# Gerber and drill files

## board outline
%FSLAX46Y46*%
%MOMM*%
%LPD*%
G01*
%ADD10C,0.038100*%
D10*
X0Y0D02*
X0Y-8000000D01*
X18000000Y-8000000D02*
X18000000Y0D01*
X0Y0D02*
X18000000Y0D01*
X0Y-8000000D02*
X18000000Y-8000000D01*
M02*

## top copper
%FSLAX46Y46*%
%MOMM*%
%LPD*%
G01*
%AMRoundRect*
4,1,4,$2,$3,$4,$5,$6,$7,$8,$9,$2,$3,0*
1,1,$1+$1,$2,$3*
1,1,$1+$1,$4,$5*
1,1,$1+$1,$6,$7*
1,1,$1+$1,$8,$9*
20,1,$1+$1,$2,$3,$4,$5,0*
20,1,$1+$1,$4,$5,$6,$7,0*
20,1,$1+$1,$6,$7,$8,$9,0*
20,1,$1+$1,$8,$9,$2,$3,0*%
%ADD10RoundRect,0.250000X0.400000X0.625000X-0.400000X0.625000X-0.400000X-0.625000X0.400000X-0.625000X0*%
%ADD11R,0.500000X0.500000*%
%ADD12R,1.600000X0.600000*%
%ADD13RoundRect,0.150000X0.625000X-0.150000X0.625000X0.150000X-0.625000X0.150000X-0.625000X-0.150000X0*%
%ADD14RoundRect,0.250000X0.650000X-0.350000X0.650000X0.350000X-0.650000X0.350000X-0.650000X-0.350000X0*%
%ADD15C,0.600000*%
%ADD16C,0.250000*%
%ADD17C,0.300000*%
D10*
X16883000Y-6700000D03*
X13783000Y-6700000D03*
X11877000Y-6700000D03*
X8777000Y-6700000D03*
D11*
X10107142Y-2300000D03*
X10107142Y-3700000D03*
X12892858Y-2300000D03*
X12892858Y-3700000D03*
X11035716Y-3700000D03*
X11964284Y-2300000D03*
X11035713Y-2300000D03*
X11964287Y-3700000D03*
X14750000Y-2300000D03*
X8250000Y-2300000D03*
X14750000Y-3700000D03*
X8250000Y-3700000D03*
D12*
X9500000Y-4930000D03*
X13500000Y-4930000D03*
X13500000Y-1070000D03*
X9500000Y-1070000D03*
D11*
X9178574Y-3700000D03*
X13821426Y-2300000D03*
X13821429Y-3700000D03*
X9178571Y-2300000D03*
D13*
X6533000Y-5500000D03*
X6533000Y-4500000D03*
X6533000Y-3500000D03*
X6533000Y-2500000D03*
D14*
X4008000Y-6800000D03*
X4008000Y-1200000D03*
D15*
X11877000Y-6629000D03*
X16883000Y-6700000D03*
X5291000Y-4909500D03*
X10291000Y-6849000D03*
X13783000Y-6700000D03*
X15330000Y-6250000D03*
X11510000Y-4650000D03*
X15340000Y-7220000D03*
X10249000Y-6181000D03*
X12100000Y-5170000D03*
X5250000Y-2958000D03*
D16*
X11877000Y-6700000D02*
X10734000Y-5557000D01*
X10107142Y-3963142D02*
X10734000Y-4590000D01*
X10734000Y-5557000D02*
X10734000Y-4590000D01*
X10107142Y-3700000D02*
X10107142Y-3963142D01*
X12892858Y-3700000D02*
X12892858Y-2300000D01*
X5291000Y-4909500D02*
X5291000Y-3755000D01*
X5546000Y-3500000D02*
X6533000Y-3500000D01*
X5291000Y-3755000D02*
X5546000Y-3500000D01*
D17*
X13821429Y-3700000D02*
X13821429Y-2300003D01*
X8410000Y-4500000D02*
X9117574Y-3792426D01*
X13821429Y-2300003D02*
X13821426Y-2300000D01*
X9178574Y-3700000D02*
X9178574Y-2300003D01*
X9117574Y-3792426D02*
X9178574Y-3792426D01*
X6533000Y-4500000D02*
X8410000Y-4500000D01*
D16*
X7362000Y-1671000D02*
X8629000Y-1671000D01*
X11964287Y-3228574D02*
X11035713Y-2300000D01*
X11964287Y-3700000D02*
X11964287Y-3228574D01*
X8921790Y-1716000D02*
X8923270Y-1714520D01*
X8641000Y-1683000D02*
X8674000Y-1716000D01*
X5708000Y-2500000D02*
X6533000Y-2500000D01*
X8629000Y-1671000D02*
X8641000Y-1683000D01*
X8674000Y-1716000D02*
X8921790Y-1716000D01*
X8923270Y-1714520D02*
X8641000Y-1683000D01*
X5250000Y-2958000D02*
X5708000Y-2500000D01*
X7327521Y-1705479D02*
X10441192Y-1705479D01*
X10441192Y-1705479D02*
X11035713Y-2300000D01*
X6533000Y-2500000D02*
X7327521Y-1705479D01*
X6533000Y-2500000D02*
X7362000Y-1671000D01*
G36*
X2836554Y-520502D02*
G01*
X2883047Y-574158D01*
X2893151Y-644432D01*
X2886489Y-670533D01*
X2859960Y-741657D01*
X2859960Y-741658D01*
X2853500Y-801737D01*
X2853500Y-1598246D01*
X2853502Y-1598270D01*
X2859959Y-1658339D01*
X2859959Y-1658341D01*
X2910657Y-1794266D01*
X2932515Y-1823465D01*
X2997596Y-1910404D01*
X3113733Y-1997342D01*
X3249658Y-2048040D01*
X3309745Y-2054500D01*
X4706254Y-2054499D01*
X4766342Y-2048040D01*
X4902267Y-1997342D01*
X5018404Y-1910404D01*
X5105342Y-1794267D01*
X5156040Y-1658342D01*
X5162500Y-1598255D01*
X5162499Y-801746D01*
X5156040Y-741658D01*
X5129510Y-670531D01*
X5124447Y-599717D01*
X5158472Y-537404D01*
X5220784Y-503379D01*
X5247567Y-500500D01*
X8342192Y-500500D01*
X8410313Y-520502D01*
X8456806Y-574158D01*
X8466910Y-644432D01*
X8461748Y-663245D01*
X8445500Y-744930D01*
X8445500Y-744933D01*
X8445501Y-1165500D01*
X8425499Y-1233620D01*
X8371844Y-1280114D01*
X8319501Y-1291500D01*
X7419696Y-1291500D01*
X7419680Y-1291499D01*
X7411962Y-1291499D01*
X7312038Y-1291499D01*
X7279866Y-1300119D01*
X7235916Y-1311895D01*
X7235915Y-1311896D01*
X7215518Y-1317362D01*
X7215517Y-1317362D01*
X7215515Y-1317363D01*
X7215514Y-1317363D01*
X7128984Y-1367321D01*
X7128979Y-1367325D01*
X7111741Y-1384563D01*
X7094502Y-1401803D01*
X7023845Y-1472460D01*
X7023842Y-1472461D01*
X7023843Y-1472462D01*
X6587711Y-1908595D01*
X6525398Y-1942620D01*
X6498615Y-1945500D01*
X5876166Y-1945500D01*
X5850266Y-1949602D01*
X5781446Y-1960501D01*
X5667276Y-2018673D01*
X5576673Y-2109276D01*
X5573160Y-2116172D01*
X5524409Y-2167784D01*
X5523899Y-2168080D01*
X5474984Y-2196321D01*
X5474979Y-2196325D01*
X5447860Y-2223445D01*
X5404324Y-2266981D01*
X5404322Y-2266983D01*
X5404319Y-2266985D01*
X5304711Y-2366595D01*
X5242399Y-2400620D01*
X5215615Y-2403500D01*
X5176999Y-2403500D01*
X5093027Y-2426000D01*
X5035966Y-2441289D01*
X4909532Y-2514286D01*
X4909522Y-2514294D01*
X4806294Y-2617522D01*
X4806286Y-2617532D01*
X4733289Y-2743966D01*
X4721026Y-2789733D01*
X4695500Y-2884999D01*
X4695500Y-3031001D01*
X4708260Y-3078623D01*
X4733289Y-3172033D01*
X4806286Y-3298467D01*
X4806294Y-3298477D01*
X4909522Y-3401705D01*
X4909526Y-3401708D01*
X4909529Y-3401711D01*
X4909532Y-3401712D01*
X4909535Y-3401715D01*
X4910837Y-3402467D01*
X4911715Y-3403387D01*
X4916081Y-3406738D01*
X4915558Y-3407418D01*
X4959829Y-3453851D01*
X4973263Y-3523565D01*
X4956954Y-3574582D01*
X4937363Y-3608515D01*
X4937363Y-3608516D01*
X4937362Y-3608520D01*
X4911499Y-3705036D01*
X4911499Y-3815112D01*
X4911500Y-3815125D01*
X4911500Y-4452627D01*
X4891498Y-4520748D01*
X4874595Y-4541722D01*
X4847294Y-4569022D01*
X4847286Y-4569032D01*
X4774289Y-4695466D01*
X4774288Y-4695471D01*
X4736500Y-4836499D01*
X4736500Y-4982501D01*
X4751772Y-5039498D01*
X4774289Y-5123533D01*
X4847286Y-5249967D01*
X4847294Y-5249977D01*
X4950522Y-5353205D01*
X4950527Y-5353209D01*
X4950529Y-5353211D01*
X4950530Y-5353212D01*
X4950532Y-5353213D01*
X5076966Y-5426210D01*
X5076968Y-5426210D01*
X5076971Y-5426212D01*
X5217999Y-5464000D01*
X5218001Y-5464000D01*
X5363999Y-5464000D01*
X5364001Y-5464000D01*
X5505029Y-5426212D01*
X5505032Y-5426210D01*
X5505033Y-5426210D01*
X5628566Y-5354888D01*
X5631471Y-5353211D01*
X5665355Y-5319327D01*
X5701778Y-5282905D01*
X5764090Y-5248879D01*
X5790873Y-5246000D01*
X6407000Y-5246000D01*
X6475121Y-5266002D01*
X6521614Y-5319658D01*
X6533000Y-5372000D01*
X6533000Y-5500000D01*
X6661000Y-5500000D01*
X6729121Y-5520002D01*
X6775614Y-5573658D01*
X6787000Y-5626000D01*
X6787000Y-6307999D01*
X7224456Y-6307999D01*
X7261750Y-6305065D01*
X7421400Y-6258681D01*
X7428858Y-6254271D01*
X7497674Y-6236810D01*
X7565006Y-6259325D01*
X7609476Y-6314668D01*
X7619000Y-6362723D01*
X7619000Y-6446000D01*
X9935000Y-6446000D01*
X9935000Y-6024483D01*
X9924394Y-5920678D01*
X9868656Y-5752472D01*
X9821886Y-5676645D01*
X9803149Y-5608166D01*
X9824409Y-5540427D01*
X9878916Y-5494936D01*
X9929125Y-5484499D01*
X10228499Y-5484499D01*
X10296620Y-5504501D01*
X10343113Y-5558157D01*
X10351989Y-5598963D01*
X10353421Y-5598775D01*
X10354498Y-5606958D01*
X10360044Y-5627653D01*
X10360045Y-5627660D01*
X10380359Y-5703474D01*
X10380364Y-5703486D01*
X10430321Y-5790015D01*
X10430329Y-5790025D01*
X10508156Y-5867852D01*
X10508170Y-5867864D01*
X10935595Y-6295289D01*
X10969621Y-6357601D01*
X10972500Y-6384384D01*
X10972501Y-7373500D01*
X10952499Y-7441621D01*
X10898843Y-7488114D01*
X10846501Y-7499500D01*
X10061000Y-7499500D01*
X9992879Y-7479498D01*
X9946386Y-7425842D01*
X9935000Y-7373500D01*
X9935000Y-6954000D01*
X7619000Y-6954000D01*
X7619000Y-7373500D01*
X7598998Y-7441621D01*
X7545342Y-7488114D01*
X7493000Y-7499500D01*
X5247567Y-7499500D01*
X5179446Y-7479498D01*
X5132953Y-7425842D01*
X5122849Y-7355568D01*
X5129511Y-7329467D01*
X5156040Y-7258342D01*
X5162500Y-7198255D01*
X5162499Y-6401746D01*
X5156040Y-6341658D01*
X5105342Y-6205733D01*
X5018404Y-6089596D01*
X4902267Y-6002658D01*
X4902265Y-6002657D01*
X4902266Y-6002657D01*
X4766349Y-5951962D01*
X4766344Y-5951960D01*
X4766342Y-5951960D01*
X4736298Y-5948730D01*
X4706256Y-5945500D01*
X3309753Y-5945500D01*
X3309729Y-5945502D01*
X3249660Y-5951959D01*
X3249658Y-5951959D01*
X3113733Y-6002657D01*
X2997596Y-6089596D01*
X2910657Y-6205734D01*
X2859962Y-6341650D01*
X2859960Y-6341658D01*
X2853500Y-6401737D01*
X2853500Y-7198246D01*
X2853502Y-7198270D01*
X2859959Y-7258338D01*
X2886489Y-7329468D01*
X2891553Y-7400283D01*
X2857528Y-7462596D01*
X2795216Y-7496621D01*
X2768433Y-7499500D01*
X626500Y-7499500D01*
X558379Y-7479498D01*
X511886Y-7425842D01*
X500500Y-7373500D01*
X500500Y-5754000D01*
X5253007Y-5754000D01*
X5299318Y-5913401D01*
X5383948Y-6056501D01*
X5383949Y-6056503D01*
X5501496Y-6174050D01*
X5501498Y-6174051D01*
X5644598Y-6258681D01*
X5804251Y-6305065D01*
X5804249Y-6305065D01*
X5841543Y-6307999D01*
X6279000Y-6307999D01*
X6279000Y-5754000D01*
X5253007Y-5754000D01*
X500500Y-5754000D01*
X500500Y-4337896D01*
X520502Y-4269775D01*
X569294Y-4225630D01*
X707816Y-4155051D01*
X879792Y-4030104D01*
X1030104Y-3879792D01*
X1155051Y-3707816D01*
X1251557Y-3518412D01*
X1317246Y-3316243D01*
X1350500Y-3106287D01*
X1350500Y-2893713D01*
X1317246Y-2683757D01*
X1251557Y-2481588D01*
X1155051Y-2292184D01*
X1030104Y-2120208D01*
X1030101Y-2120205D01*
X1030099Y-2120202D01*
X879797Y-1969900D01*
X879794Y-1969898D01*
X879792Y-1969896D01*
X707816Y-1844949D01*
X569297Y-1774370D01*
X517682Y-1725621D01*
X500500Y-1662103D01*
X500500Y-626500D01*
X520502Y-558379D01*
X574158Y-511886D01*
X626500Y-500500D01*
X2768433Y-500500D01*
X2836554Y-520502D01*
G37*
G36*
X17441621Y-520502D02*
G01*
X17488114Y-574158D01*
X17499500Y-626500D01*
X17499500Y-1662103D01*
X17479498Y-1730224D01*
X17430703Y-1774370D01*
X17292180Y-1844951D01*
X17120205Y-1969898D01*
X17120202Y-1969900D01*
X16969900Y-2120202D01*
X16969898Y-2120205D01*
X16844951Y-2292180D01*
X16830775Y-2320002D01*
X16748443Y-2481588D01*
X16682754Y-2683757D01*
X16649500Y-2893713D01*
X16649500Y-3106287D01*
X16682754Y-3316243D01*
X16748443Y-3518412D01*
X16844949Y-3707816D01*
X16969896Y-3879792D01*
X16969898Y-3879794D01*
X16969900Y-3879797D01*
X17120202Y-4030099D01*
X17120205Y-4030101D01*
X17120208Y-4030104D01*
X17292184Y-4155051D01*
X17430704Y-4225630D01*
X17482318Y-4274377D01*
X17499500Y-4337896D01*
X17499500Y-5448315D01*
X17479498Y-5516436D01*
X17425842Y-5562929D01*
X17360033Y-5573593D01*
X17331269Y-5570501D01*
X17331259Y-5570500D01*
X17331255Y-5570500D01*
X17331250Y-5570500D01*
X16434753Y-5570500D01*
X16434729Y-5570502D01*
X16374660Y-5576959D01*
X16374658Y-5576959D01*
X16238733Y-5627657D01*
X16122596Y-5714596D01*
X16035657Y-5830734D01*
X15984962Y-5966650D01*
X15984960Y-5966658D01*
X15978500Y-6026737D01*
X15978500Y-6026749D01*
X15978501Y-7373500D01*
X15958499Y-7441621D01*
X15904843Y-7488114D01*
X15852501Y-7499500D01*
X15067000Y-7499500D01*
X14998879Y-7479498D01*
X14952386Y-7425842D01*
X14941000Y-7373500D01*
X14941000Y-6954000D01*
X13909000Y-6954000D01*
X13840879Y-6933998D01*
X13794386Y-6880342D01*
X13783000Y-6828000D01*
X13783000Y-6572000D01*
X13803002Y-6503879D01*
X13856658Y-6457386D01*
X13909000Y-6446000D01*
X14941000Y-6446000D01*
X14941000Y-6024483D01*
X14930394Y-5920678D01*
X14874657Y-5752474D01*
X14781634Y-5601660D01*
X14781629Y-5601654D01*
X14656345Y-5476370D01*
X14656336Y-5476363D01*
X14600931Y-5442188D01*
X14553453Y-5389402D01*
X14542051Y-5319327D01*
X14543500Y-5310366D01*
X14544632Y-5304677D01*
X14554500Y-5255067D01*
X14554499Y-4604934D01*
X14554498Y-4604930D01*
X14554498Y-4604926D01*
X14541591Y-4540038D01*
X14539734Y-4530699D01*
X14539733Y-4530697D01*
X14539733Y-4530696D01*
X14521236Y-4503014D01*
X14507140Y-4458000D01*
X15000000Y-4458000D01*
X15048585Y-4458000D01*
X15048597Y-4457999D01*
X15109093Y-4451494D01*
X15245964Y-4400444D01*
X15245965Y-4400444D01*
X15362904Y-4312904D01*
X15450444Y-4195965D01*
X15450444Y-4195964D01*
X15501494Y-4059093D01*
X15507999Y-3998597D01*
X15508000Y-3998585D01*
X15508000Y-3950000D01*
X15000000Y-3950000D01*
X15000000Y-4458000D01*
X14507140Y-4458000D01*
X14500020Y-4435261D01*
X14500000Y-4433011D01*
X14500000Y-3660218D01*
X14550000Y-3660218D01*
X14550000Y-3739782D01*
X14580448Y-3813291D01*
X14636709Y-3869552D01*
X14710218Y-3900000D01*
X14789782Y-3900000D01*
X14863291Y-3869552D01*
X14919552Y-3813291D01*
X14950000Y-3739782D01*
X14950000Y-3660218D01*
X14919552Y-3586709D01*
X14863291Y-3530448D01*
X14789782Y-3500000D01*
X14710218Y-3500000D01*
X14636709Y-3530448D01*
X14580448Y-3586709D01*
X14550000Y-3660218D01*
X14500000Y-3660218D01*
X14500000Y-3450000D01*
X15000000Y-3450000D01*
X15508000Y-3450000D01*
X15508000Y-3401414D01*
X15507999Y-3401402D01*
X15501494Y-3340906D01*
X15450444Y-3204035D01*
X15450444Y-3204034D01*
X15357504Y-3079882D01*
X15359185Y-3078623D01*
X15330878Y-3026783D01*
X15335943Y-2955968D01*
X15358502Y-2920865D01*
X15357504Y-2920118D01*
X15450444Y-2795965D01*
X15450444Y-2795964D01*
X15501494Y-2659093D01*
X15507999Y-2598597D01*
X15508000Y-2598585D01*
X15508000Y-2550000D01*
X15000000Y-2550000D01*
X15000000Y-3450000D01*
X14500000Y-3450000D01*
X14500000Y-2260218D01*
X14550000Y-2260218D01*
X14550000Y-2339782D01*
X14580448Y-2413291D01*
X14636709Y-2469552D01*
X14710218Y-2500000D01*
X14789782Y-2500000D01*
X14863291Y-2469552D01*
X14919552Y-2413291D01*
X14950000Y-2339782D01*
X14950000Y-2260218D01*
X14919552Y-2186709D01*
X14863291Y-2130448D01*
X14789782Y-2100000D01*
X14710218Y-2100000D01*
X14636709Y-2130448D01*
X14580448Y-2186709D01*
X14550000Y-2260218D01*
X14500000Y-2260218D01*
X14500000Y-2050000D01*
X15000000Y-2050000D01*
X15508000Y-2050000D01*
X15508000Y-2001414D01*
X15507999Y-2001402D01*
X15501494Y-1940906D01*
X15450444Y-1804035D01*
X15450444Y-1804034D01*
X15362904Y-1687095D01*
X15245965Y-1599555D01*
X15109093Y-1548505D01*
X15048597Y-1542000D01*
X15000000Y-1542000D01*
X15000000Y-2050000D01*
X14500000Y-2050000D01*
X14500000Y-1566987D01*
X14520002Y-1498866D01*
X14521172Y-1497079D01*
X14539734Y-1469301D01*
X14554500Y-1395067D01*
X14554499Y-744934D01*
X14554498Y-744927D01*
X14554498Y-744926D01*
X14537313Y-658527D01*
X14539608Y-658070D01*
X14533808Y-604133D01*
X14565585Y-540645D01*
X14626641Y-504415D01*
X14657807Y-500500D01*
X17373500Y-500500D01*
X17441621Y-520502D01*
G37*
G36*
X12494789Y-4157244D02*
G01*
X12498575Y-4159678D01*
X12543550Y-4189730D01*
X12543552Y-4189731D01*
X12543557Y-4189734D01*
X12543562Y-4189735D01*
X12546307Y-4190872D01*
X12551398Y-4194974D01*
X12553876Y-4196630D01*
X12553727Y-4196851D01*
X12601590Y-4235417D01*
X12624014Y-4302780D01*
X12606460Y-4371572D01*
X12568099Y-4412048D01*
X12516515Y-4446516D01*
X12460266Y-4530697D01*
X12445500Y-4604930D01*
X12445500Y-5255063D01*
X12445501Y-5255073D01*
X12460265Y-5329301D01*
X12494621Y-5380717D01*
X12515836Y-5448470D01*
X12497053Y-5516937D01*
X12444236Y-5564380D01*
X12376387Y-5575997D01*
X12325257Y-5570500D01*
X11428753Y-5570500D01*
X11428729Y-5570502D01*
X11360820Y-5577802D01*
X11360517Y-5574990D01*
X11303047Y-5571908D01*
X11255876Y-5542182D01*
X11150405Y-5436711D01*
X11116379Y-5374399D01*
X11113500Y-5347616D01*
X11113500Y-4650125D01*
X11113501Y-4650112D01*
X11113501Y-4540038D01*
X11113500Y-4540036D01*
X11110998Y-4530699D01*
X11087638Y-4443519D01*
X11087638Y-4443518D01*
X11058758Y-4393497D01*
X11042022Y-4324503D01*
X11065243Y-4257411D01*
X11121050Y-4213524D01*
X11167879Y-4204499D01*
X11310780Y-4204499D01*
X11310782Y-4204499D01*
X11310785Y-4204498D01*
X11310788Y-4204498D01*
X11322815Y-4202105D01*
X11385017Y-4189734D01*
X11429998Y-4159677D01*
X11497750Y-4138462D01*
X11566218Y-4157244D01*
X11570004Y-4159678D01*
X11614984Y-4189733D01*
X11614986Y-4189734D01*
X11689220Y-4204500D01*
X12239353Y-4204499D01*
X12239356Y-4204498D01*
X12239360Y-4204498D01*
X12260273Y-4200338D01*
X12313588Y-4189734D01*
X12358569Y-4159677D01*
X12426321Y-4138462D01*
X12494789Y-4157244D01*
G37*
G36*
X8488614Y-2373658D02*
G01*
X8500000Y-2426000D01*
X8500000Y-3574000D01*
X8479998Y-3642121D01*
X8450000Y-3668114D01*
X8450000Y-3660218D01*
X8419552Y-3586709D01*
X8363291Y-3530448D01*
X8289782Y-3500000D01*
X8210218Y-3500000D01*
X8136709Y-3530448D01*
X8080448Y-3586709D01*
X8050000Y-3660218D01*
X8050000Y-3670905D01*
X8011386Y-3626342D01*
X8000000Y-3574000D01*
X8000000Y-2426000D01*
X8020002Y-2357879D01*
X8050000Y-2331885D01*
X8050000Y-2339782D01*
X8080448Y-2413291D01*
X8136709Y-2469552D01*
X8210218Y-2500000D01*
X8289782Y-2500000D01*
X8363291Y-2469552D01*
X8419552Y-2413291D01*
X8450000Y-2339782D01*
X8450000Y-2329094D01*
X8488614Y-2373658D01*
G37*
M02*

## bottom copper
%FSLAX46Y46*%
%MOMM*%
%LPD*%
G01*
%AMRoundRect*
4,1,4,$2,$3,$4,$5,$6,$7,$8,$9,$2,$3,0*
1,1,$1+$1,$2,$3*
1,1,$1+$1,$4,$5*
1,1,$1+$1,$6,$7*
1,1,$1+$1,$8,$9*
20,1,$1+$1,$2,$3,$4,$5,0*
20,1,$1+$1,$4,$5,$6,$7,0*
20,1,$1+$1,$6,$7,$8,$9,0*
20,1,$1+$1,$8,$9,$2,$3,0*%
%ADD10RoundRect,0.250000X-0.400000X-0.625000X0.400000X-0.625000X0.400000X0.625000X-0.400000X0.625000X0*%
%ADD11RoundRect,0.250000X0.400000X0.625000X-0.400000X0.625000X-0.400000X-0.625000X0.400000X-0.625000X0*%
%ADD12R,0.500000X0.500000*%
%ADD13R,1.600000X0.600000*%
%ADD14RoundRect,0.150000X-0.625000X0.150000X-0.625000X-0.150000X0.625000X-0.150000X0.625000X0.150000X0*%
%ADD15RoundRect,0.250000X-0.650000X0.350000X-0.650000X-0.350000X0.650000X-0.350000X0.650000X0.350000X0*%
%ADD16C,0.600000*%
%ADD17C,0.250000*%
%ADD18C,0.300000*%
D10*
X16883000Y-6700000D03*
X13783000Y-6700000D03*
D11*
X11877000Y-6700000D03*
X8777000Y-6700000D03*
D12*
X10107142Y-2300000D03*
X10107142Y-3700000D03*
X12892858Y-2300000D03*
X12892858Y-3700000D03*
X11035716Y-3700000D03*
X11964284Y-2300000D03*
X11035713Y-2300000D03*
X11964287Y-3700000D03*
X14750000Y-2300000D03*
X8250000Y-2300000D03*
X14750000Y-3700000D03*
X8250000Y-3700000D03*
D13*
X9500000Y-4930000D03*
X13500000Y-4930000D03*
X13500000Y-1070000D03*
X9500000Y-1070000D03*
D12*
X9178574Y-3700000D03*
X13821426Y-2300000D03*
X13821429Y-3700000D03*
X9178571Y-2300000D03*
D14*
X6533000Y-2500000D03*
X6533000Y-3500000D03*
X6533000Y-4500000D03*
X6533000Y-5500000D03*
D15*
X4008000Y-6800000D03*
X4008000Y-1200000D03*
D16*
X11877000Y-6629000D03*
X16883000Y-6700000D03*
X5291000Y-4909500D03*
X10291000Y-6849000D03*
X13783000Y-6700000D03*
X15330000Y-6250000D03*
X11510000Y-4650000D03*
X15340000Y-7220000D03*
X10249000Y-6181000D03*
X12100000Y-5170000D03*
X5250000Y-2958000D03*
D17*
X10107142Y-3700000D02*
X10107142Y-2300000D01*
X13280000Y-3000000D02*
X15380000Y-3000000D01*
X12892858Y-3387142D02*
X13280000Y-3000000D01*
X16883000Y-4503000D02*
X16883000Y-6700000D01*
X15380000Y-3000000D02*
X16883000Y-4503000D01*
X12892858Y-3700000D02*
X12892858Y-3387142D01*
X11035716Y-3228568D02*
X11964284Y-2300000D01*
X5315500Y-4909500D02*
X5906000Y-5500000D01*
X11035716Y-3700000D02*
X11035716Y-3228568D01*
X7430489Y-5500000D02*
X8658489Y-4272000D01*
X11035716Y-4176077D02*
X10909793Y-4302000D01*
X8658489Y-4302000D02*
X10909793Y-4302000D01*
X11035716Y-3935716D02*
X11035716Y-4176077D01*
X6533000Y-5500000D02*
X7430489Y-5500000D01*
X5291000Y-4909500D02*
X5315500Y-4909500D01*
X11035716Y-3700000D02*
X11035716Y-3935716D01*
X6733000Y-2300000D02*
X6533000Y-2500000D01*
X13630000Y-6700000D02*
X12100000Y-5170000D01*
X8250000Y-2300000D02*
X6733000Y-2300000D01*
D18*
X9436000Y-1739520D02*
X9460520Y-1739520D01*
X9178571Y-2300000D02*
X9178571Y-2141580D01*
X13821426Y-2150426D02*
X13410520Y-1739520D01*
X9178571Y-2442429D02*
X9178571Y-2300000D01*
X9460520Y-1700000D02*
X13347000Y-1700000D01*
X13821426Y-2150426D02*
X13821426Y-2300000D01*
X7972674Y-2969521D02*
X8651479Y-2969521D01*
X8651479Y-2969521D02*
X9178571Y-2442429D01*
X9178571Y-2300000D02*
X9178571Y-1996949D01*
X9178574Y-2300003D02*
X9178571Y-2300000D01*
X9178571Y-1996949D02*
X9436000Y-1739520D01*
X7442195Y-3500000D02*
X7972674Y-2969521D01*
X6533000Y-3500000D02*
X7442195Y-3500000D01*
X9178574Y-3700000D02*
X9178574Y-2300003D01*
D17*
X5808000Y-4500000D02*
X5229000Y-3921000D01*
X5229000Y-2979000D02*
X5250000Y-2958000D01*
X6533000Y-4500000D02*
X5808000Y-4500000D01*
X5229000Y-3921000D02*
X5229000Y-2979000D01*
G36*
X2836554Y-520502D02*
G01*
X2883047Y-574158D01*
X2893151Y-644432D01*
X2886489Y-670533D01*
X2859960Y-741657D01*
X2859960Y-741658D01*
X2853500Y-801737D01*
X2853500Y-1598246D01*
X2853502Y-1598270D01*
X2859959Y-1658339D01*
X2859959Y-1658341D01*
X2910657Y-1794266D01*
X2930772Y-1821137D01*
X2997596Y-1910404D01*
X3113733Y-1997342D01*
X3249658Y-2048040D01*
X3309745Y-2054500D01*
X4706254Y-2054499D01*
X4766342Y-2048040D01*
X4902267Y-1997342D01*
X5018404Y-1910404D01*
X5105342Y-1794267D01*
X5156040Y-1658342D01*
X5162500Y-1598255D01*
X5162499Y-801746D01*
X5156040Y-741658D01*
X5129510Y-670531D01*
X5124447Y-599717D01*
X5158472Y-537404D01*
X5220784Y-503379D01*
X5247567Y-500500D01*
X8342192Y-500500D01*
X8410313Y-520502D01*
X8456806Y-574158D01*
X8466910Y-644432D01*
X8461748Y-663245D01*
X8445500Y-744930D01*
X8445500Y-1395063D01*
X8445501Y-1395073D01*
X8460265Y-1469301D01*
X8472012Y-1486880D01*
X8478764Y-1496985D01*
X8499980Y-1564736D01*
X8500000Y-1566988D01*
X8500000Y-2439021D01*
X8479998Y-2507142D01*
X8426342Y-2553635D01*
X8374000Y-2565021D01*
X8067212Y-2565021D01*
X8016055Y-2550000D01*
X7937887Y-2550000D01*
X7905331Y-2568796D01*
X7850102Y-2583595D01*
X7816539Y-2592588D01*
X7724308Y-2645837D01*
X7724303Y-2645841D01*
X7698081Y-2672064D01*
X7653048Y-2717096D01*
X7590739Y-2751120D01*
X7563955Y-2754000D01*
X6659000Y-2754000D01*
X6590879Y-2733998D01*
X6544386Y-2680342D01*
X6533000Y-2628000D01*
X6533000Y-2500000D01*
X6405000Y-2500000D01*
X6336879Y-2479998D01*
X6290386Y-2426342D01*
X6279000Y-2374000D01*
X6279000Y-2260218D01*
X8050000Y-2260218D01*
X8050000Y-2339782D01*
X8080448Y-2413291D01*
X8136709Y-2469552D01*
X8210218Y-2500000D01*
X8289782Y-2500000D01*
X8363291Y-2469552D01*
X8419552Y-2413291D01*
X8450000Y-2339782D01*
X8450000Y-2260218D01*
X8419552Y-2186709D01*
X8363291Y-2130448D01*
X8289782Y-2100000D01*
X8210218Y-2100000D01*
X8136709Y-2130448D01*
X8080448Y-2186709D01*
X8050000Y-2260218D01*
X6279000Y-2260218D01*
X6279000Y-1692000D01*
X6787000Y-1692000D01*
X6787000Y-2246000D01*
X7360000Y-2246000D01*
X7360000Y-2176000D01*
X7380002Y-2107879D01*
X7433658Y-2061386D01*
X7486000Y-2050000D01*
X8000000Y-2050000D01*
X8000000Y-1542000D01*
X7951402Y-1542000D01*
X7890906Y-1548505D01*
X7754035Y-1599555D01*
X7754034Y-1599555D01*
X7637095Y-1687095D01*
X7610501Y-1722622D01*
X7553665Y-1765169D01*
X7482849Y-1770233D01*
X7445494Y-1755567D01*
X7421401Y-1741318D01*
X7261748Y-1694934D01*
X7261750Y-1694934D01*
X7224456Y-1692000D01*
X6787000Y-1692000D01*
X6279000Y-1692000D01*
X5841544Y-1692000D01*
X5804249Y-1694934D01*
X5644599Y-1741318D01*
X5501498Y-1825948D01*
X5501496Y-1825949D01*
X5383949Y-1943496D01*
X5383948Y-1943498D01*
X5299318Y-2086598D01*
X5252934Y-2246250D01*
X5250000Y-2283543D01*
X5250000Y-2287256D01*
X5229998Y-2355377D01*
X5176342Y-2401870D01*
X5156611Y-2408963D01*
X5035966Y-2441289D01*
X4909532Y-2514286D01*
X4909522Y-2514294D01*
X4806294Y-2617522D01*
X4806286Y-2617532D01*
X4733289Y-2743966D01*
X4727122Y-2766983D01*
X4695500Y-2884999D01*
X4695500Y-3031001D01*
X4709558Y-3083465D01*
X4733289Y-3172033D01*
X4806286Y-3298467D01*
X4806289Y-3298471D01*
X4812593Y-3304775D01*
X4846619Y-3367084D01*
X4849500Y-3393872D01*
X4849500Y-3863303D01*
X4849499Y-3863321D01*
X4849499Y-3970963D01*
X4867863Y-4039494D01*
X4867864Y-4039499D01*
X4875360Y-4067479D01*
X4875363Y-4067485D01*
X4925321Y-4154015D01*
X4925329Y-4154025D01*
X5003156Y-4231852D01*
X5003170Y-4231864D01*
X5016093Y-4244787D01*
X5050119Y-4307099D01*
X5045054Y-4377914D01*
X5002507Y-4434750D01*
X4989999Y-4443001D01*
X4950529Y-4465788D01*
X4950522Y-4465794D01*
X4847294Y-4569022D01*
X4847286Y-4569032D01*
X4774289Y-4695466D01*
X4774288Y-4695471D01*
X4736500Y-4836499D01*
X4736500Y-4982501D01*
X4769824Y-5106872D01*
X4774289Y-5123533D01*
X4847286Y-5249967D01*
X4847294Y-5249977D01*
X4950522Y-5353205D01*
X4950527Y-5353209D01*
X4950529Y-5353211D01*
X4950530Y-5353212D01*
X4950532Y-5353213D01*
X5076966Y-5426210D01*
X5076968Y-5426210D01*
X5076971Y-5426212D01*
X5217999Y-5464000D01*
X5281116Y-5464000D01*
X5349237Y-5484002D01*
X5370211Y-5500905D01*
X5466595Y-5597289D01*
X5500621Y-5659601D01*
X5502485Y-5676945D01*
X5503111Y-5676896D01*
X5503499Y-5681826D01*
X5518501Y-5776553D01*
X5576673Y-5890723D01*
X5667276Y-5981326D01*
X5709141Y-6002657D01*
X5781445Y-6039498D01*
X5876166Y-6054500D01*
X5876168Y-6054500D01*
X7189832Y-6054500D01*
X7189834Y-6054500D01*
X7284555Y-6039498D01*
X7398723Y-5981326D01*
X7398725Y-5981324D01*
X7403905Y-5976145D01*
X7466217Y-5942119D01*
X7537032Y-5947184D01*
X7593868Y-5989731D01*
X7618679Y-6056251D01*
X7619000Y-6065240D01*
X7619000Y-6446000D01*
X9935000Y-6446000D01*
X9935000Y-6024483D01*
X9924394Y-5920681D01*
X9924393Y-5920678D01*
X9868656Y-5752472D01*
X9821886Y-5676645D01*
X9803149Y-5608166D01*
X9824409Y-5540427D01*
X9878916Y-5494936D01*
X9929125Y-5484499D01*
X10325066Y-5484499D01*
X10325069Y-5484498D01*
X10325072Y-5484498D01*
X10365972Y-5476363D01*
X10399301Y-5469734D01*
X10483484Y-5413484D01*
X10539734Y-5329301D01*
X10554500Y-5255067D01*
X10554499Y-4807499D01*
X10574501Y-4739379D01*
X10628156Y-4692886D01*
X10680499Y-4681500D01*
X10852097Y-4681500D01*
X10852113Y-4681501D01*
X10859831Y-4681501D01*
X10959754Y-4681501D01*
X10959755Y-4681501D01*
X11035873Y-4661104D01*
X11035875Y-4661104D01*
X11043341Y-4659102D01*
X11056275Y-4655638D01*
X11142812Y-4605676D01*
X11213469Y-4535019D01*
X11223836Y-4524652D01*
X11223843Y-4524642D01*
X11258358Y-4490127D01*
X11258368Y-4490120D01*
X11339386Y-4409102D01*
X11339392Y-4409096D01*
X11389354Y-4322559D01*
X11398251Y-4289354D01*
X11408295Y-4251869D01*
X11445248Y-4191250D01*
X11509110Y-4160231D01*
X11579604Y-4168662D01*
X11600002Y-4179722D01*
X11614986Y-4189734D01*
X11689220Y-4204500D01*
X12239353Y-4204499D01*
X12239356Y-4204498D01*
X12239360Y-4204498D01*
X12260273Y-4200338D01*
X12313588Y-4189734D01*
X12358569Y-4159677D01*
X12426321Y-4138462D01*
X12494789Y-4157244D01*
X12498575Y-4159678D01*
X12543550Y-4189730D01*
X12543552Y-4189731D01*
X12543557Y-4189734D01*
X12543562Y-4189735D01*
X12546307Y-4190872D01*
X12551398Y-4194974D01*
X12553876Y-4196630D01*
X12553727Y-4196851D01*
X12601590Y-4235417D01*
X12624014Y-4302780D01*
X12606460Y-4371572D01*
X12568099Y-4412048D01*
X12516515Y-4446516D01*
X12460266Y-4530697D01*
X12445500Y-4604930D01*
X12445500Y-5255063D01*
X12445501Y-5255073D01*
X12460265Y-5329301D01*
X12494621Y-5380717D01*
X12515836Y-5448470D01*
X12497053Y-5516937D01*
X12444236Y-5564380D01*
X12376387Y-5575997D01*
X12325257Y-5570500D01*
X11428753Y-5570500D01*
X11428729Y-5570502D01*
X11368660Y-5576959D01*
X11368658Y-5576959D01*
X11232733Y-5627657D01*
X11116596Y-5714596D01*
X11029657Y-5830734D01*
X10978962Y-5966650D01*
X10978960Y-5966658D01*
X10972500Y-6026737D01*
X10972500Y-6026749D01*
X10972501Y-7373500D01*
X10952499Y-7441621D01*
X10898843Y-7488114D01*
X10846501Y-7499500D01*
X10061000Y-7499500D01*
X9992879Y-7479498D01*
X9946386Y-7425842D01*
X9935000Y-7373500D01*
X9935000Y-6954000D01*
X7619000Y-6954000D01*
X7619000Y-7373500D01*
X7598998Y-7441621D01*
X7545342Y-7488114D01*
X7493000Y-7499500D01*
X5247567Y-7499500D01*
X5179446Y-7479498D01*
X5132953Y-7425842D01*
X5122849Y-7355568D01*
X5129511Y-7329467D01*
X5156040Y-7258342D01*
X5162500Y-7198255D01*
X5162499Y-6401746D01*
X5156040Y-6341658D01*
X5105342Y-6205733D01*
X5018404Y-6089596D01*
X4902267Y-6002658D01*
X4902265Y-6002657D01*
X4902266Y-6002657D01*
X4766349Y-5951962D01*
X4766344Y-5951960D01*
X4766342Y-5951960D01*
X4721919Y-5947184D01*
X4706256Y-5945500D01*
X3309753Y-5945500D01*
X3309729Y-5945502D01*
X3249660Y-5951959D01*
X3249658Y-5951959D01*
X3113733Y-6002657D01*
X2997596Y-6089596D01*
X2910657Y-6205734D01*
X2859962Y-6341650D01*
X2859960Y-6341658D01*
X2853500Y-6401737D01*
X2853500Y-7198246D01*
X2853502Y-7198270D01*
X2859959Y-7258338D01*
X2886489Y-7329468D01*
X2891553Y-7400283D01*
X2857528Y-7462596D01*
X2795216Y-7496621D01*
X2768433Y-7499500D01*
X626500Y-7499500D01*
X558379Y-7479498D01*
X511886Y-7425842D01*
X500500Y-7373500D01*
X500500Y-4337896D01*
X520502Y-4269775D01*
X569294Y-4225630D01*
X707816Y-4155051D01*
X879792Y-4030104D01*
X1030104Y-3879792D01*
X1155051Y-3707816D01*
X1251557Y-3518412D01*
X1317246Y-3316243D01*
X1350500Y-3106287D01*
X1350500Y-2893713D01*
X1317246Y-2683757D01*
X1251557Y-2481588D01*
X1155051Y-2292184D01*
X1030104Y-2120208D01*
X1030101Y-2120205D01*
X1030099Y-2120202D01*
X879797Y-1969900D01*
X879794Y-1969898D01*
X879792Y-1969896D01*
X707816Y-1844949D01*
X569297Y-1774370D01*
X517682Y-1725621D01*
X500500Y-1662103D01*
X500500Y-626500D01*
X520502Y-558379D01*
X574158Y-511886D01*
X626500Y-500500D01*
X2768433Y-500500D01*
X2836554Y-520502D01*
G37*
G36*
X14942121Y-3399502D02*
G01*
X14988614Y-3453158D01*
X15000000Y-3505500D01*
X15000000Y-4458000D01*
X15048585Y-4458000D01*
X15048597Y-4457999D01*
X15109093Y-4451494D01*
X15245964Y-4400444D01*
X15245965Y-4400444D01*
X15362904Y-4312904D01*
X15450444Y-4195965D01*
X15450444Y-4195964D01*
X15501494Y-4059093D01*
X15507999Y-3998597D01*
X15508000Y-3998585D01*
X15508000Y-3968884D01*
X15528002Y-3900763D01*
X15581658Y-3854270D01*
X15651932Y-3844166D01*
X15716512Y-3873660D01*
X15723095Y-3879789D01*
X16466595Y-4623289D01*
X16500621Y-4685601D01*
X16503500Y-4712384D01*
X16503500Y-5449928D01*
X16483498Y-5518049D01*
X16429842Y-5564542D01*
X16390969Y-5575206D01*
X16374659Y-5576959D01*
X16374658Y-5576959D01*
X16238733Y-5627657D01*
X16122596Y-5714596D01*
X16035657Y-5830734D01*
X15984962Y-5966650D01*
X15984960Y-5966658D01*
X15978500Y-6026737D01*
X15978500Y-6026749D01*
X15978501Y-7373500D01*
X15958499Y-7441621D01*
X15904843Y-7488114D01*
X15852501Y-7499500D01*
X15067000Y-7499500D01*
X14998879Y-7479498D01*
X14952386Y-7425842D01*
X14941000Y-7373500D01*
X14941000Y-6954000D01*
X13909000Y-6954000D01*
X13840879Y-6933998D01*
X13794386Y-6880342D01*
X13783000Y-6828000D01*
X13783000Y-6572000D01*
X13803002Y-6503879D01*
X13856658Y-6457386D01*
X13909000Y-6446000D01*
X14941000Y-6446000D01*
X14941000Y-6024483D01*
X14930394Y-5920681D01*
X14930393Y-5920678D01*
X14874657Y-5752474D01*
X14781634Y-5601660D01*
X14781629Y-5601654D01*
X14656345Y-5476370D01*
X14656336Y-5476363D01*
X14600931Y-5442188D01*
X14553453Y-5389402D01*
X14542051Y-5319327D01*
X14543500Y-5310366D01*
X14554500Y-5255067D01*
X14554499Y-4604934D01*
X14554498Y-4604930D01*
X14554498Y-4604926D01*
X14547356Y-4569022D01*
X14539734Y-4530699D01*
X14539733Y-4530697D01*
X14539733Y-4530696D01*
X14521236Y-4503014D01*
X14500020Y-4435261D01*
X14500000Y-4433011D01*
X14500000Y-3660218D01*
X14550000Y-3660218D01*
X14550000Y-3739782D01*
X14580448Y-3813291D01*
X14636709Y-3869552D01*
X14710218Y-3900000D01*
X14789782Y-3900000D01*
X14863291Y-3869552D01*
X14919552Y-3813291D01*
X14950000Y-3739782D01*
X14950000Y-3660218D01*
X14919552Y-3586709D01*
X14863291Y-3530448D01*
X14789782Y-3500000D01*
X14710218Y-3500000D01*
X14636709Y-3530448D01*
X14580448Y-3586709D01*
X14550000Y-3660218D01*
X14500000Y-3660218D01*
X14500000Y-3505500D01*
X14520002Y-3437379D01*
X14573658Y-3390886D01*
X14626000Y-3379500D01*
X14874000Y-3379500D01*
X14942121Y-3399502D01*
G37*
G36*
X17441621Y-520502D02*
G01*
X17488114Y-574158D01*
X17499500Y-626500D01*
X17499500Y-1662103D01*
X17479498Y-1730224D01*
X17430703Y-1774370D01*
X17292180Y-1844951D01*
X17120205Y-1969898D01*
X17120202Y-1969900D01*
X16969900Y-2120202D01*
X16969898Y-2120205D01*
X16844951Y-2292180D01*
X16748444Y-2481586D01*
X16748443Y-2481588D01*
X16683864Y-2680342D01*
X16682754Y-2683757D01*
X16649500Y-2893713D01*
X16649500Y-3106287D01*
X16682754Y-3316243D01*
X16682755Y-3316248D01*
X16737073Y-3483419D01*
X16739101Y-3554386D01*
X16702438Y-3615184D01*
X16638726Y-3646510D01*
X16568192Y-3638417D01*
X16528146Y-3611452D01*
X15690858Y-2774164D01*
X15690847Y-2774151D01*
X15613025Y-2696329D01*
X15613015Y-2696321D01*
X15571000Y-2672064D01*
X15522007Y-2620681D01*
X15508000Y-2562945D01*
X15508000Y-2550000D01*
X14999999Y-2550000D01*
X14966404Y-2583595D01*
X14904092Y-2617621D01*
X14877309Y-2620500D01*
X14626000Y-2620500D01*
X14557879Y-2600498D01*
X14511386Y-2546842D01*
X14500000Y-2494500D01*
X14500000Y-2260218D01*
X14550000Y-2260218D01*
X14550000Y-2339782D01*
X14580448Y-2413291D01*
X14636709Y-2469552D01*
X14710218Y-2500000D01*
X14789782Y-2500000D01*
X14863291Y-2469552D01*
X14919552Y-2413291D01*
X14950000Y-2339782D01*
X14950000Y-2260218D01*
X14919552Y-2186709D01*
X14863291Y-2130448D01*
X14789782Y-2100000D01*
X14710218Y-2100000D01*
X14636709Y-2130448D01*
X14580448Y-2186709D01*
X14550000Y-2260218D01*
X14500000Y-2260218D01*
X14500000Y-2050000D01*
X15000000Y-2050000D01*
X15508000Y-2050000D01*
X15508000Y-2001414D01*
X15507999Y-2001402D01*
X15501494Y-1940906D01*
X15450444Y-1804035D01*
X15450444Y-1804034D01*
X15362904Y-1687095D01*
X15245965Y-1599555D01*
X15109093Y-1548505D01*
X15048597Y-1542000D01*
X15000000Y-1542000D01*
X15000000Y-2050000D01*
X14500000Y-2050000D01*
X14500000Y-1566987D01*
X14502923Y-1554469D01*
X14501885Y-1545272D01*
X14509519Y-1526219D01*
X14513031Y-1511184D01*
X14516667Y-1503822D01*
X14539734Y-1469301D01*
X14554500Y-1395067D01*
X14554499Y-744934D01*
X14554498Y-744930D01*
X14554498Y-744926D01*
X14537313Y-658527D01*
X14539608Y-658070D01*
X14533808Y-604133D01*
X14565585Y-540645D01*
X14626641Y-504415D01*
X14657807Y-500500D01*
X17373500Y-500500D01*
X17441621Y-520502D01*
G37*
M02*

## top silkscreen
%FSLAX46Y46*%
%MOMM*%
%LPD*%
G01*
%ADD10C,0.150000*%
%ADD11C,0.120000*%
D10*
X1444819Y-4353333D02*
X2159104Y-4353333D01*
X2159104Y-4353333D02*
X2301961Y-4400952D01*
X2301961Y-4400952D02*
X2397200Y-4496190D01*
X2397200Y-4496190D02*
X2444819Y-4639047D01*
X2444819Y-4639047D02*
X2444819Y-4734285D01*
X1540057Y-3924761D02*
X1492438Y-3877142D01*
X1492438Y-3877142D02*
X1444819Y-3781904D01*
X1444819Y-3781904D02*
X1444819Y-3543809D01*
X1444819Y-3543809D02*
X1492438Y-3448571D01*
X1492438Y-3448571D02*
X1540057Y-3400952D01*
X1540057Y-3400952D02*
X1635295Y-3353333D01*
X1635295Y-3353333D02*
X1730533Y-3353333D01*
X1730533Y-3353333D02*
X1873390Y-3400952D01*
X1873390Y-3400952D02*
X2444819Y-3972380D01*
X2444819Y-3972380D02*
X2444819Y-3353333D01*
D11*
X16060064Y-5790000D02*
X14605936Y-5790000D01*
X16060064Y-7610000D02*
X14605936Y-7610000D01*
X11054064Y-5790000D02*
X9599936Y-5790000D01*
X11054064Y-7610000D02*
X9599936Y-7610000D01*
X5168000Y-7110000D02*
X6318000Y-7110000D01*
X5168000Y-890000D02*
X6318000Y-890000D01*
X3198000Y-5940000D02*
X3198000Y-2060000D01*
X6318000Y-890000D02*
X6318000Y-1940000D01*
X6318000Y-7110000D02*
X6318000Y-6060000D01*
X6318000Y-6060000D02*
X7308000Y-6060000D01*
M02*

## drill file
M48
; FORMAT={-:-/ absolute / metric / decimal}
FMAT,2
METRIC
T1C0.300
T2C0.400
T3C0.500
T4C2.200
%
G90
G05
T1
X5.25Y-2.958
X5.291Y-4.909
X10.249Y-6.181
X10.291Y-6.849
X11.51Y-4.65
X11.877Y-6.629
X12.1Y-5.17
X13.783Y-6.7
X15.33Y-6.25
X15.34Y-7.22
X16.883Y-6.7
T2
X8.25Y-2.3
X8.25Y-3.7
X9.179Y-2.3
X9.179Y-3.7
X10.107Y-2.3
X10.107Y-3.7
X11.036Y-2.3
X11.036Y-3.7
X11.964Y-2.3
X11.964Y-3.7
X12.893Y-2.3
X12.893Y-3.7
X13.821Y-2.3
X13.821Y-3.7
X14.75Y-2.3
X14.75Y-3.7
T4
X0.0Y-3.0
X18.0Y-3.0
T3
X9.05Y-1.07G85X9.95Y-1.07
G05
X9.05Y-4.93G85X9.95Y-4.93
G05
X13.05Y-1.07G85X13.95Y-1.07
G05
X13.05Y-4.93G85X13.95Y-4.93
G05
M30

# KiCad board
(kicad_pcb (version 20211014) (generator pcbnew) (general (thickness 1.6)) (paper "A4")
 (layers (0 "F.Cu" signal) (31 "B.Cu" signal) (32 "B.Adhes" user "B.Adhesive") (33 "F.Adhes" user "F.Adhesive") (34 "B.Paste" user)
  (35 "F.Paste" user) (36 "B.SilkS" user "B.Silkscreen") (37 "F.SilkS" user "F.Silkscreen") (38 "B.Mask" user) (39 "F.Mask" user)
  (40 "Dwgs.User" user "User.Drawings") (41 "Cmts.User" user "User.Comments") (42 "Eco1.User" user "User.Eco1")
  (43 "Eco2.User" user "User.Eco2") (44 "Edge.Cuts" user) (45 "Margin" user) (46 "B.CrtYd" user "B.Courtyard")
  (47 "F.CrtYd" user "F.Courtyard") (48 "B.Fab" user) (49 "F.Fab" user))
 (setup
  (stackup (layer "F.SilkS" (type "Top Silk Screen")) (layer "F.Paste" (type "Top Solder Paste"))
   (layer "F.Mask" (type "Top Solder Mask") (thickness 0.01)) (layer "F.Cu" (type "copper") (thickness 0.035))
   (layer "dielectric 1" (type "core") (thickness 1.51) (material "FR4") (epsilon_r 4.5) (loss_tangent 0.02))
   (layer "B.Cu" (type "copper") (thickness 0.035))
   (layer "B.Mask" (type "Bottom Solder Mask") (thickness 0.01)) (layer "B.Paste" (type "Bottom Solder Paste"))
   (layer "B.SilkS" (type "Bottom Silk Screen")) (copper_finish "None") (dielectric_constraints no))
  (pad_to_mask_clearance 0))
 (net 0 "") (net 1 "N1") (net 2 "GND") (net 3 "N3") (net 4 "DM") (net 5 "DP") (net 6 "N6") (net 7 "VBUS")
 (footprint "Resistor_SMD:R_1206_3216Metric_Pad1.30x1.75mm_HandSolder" (layer "F.Cu") (at 15.333 6.7 180)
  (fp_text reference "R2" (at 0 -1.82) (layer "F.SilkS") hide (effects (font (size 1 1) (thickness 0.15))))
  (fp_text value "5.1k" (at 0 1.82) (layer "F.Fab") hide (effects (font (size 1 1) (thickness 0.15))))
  (fp_line (start -0.727064 0.91) (end 0.727064 0.91) (layer "F.SilkS") (width 0.12))
  (fp_line (start -0.727064 -0.91) (end 0.727064 -0.91) (layer "F.SilkS") (width 0.12))
  (pad "1" smd roundrect (at -1.55 0) (size 1.3 1.75) (layers "B.Cu" "B.Paste" "B.Mask") (roundrect_rratio 0.192308) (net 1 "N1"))
  (pad "1" smd roundrect (at -1.55 0 180) (size 1.3 1.75) (layers "F.Cu" "F.Paste" "F.Mask") (roundrect_rratio 0.192308) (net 1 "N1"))
  (pad "2" smd roundrect (at 1.55 0) (size 1.3 1.75) (layers "B.Cu" "B.Paste" "B.Mask") (roundrect_rratio 0.192308) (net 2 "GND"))
  (pad "2" smd roundrect (at 1.55 0 180) (size 1.3 1.75) (layers "F.Cu" "F.Paste" "F.Mask") (roundrect_rratio 0.192308) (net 2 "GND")))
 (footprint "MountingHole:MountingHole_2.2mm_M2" (layer "F.Cu") (at 18 3)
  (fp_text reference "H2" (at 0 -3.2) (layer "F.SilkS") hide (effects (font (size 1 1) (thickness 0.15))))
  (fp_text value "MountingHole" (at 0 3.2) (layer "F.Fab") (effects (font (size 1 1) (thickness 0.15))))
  (pad "" np_thru_hole circle (at 0 0) (size 2.2 2.2) (drill 2.2) (layers *.Cu *.Mask)))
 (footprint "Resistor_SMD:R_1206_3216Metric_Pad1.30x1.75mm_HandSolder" (layer "F.Cu") (at 10.327 6.7 180)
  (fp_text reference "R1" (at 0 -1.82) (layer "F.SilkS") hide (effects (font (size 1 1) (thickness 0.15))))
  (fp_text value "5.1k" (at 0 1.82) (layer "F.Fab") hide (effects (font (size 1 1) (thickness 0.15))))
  (fp_line (start -0.727064 0.91) (end 0.727064 0.91) (layer "F.SilkS") (width 0.12))
  (fp_line (start -0.727064 -0.91) (end 0.727064 -0.91) (layer "F.SilkS") (width 0.12))
  (pad "1" smd roundrect (at -1.55 0 180) (size 1.3 1.75) (layers "B.Cu" "B.Paste" "B.Mask") (roundrect_rratio 0.192308) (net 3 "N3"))
  (pad "1" smd roundrect (at -1.55 0 180) (size 1.3 1.75) (layers "F.Cu" "F.Paste" "F.Mask") (roundrect_rratio 0.192308) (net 3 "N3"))
  (pad "2" smd roundrect (at 1.55 0 180) (size 1.3 1.75) (layers "F.Cu" "F.Paste" "F.Mask") (roundrect_rratio 0.192308) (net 2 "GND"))
  (pad "2" smd roundrect (at 1.55 0 180) (size 1.3 1.75) (layers "B.Cu" "B.Paste" "B.Mask") (roundrect_rratio 0.192308) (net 2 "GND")))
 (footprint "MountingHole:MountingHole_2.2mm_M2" (layer "F.Cu") (at 0 3)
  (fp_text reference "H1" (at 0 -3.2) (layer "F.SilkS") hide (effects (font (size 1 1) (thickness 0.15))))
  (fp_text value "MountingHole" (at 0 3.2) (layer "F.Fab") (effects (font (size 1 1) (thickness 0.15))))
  (pad "" np_thru_hole circle (at 0 0) (size 2.2 2.2) (drill 2.2) (layers *.Cu *.Mask)))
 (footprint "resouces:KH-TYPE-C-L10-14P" (layer "F.Cu") (at 11.5 3)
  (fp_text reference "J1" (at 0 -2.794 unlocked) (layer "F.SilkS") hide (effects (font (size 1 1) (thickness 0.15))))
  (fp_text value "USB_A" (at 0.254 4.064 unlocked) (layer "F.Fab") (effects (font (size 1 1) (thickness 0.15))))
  (pad "CC1" thru_hole rect (at -1.392858 -0.7) (size 0.5 0.5) (drill oval 0.4) (layers *.Cu *.Mask) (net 3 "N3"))
  (pad "CC1" thru_hole rect (at -1.392858 0.7) (size 0.5 0.5) (drill oval 0.4) (layers *.Cu *.Mask) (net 3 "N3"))
  (pad "CC2" thru_hole rect (at 1.392858 -0.7) (size 0.5 0.5) (drill oval 0.4) (layers *.Cu *.Mask) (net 1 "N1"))
  (pad "CC2" thru_hole rect (at 1.392858 0.7) (size 0.5 0.5) (drill oval 0.4) (layers *.Cu *.Mask) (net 1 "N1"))
  (pad "DM" thru_hole rect (at -0.464284 0.7) (size 0.5 0.5) (drill oval 0.4) (layers *.Cu *.Mask) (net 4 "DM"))
  (pad "DM" thru_hole rect (at 0.464284 -0.7) (size 0.5 0.5) (drill oval 0.4) (layers *.Cu *.Mask) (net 4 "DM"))
  (pad "DP" thru_hole rect (at -0.464287 -0.7) (size 0.5 0.5) (drill oval 0.4) (layers *.Cu *.Mask) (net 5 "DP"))
  (pad "DP" thru_hole rect (at 0.464287 0.7) (size 0.5 0.5) (drill oval 0.4) (layers *.Cu *.Mask) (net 5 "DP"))
  (pad "G" thru_hole rect (at 3.25 -0.7) (size 0.5 0.5) (drill oval 0.4) (layers *.Cu *.Mask) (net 2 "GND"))
  (pad "G" thru_hole rect (at -3.25 -0.7) (size 0.5 0.5) (drill oval 0.4) (layers *.Cu *.Mask) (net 2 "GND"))
  (pad "G" thru_hole rect (at 3.25 0.7) (size 0.5 0.5) (drill oval 0.4) (layers *.Cu *.Mask) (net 2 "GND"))
  (pad "G" thru_hole rect (at -3.25 0.7) (size 0.5 0.5) (drill oval 0.4) (layers *.Cu *.Mask) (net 2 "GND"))
  (pad "SHIELD" thru_hole rect (at -2 1.93) (size 1.6 0.6) (drill oval 1.4 0.5) (layers *.Cu *.Mask) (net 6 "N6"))
  (pad "SHIELD" thru_hole rect (at 2 1.93) (size 1.6 0.6) (drill oval 1.4 0.5) (layers *.Cu *.Mask) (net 6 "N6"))
  (pad "SHIELD" thru_hole rect (at 2 -1.93) (size 1.6 0.6) (drill oval 1.4 0.5) (layers *.Cu *.Mask) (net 6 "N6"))
  (pad "SHIELD" thru_hole rect (at -2 -1.93) (size 1.6 0.6) (drill oval 1.4 0.5) (layers *.Cu *.Mask) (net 6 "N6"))
  (pad "VBUS" thru_hole rect (at -2.321426 0.7) (size 0.5 0.5) (drill oval 0.4) (layers *.Cu *.Mask) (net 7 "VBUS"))
  (pad "VBUS" thru_hole rect (at 2.321426 -0.7) (size 0.5 0.5) (drill oval 0.4) (layers *.Cu *.Mask) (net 7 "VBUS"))
  (pad "VBUS" thru_hole rect (at 2.321429 0.7) (size 0.5 0.5) (drill oval 0.4) (layers *.Cu *.Mask) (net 7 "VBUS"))
  (pad "VBUS" thru_hole rect (at -2.321429 -0.7) (size 0.5 0.5) (drill oval 0.4) (layers *.Cu *.Mask) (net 7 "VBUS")))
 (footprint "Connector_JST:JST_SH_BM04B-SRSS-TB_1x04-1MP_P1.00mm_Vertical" (layer "F.Cu") (at 5.208 4 90)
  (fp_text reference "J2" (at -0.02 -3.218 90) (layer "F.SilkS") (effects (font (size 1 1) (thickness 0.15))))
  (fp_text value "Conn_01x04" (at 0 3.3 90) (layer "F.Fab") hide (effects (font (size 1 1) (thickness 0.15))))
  (fp_line (start -3.11 -0.04) (end -3.11 1.11) (layer "F.SilkS") (width 0.12))
  (fp_line (start 3.11 -0.04) (end 3.11 1.11) (layer "F.SilkS") (width 0.12))
  (fp_line (start -1.94 -2.01) (end 1.94 -2.01) (layer "F.SilkS") (width 0.12))
  (fp_line (start 3.11 1.11) (end 2.06 1.11) (layer "F.SilkS") (width 0.12))
  (fp_line (start -3.11 1.11) (end -2.06 1.11) (layer "F.SilkS") (width 0.12))
  (fp_line (start -2.06 1.11) (end -2.06 2.1) (layer "F.SilkS") (width 0.12))
  (pad "1" smd roundrect (at -1.5 1.325 90) (size 0.6 1.55) (layers "F.Cu" "F.Paste" "F.Mask") (roundrect_rratio 0.25) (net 2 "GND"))
  (pad "2" smd roundrect (at -0.5 1.325 90) (size 0.6 1.55) (layers "F.Cu" "F.Paste" "F.Mask") (roundrect_rratio 0.25) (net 7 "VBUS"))
  (pad "3" smd roundrect (at 0.5 1.325 90) (size 0.6 1.55) (layers "F.Cu" "F.Paste" "F.Mask") (roundrect_rratio 0.25) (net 4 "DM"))
  (pad "4" smd roundrect (at 1.5 1.325 90) (size 0.6 1.55) (layers "F.Cu" "F.Paste" "F.Mask") (roundrect_rratio 0.25) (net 5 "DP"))
  (pad "MP" smd roundrect (at -2.8 -1.2 90) (size 1.2 1.8) (layers "F.Cu" "F.Paste" "F.Mask") (roundrect_rratio 0.208333))
  (pad "MP" smd roundrect (at 2.8 -1.2 90) (size 1.2 1.8) (layers "F.Cu" "F.Paste" "F.Mask") (roundrect_rratio 0.208333)))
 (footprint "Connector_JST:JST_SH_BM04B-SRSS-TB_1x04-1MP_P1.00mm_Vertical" (layer "B.Cu") (at 5.208 4 -90)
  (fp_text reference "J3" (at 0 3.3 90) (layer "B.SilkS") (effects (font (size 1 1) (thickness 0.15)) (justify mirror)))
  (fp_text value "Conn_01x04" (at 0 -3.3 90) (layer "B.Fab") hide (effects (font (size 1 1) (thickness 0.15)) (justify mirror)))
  (pad "1" smd roundrect (at -1.5 -1.325 270) (size 0.6 1.55) (layers "B.Cu" "B.Paste" "B.Mask") (roundrect_rratio 0.25) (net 2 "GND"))
  (pad "2" smd roundrect (at -0.5 -1.325 270) (size 0.6 1.55) (layers "B.Cu" "B.Paste" "B.Mask") (roundrect_rratio 0.25) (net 7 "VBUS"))
  (pad "3" smd roundrect (at 0.5 -1.325 270) (size 0.6 1.55) (layers "B.Cu" "B.Paste" "B.Mask") (roundrect_rratio 0.25) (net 5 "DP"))
  (pad "4" smd roundrect (at 1.5 -1.325 270) (size 0.6 1.55) (layers "B.Cu" "B.Paste" "B.Mask") (roundrect_rratio 0.25) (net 4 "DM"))
  (pad "MP" smd roundrect (at 2.8 1.2 270) (size 1.2 1.8) (layers "B.Cu" "B.Paste" "B.Mask") (roundrect_rratio 0.208333))
  (pad "MP" smd roundrect (at -2.8 1.2 270) (size 1.2 1.8) (layers "B.Cu" "B.Paste" "B.Mask") (roundrect_rratio 0.208333)))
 (gr_line (start 0 0) (end 0 8) (layer "Edge.Cuts") (width 0.0381))
 (gr_line (start 18 8) (end 18 0) (layer "Edge.Cuts") (width 0.0381))
 (gr_line (start 0 0) (end 18 0) (layer "Edge.Cuts") (width 0.0381))
 (gr_line (start 0 8) (end 18 8) (layer "Edge.Cuts") (width 0.0381))
 (segment (start 11.877 6.7) (end 10.734 5.557) (width 0.25) (layer "F.Cu") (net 3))
 (segment (start 10.107142 3.963142) (end 10.734 4.59) (width 0.25) (layer "F.Cu") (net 3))
 (segment (start 10.734 5.557) (end 10.734 4.59) (width 0.25) (layer "F.Cu") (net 3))
 (segment (start 10.107142 3.7) (end 10.107142 3.963142) (width 0.25) (layer "F.Cu") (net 3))
 (via (at 11.877 6.629) (size 0.6) (drill 0.3) (layers "F.Cu" "B.Cu") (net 3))
 (segment (start 10.107142 3.7) (end 10.107142 2.3) (width 0.25) (layer "B.Cu") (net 3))
 (segment (start 12.892858 3.7) (end 12.892858 2.3) (width 0.25) (layer "F.Cu") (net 1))
 (via (at 16.883 6.7) (size 0.6) (drill 0.3) (layers "F.Cu" "B.Cu") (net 1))
 (segment (start 13.28 3) (end 15.38 3) (width 0.25) (layer "B.Cu") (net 1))
 (segment (start 12.892858 3.387142) (end 13.28 3) (width 0.25) (layer "B.Cu") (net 1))
 (segment (start 16.883 4.503) (end 16.883 6.7) (width 0.25) (layer "B.Cu") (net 1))
 (segment (start 15.38 3) (end 16.883 4.503) (width 0.25) (layer "B.Cu") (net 1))
 (segment (start 12.892858 3.7) (end 12.892858 3.387142) (width 0.25) (layer "B.Cu") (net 1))
 (segment (start 5.291 4.9095) (end 5.291 3.755) (width 0.25) (layer "F.Cu") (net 4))
 (segment (start 5.546 3.5) (end 6.533 3.5) (width 0.25) (layer "F.Cu") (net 4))
 (segment (start 5.291 3.755) (end 5.546 3.5) (width 0.25) (layer "F.Cu") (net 4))
 (via (at 5.291 4.9095) (size 0.6) (drill 0.3) (layers "F.Cu" "B.Cu") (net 4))
 (segment (start 11.035716 3.228568) (end 11.964284 2.3) (width 0.25) (layer "B.Cu") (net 4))
 (segment (start 5.3155 4.9095) (end 5.906 5.5) (width 0.25) (layer "B.Cu") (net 4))
 (segment (start 11.035716 3.7) (end 11.035716 3.228568) (width 0.25) (layer "B.Cu") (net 4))
 (segment (start 7.430489 5.5) (end 8.658489 4.272) (width 0.25) (layer "B.Cu") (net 4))
 (segment (start 11.035716 4.176077) (end 10.909793 4.302) (width 0.25) (layer "B.Cu") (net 4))
 (segment (start 8.658489 4.302) (end 10.909793 4.302) (width 0.25) (layer "B.Cu") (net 4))
 (segment (start 11.035716 3.935716) (end 11.035716 4.176077) (width 0.25) (layer "B.Cu") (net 4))
 (segment (start 6.533 5.5) (end 7.430489 5.5) (width 0.25) (layer "B.Cu") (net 4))
 (segment (start 5.291 4.9095) (end 5.3155 4.9095) (width 0.25) (layer "B.Cu") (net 4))
 (segment (start 11.035716 3.7) (end 11.035716 3.935716) (width 0.25) (layer "B.Cu") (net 4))
 (via (at 10.291 6.849) (size 0.6) (drill 0.3) (layers "F.Cu" "B.Cu") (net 2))
 (via (at 13.783 6.7) (size 0.6) (drill 0.3) (layers "F.Cu" "B.Cu") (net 2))
 (via (at 15.33 6.25) (size 0.6) (drill 0.3) (layers "F.Cu" "B.Cu") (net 2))
 (via (at 11.51 4.65) (size 0.6) (drill 0.3) (layers "F.Cu" "B.Cu") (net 2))
 (via (at 15.34 7.22) (size 0.6) (drill 0.3) (layers "F.Cu" "B.Cu") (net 2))
 (via (at 10.249 6.181) (size 0.6) (drill 0.3) (layers "F.Cu" "B.Cu") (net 2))
 (via (at 12.1 5.17) (size 0.6) (drill 0.3) (layers "F.Cu" "B.Cu") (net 2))
 (segment (start 6.733 2.3) (end 6.533 2.5) (width 0.25) (layer "B.Cu") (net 2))
 (segment (start 13.63 6.7) (end 12.1 5.17) (width 0.25) (layer "B.Cu") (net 2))
 (segment (start 8.25 2.3) (end 6.733 2.3) (width 0.25) (layer "B.Cu") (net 2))
 (segment (start 13.821429 3.7) (end 13.821429 2.300003) (width 0.3) (layer "F.Cu") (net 7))
 (segment (start 8.41 4.5) (end 9.117574 3.792426) (width 0.3) (layer "F.Cu") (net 7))
 (segment (start 13.821429 2.300003) (end 13.821426 2.3) (width 0.3) (layer "F.Cu") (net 7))
 (segment (start 9.178574 3.7) (end 9.178574 2.300003) (width 0.3) (layer "F.Cu") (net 7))
 (segment (start 9.117574 3.792426) (end 9.178574 3.792426) (width 0.3) (layer "F.Cu") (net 7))
 (segment (start 6.533 4.5) (end 8.41 4.5) (width 0.3) (layer "F.Cu") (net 7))
 (segment (start 9.436 1.73952) (end 9.46052 1.73952) (width 0.3) (layer "B.Cu") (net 7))
 (segment (start 9.178571 2.3) (end 9.178571 2.14158) (width 0.3) (layer "B.Cu") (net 7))
 (segment (start 13.821426 2.150426) (end 13.41052 1.73952) (width 0.3) (layer "B.Cu") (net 7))
 (segment (start 9.178571 2.442429) (end 9.178571 2.3) (width 0.3) (layer "B.Cu") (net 7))
 (segment (start 9.46052 1.7) (end 13.347 1.7) (width 0.3) (layer "B.Cu") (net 7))
 (segment (start 13.821426 2.150426) (end 13.821426 2.3) (width 0.3) (layer "B.Cu") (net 7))
 (segment (start 7.972674 2.969521) (end 8.651479 2.969521) (width 0.3) (layer "B.Cu") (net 7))
 (segment (start 8.651479 2.969521) (end 9.178571 2.442429) (width 0.3) (layer "B.Cu") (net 7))
 (segment (start 9.178571 2.3) (end 9.178571 1.996949) (width 0.3) (layer "B.Cu") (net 7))
 (segment (start 9.178574 2.300003) (end 9.178571 2.3) (width 0.3) (layer "B.Cu") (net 7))
 (segment (start 9.178571 1.996949) (end 9.436 1.73952) (width 0.3) (layer "B.Cu") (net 7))
 (segment (start 7.442195 3.5) (end 7.972674 2.969521) (width 0.3) (layer "B.Cu") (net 7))
 (segment (start 6.533 3.5) (end 7.442195 3.5) (width 0.3) (layer "B.Cu") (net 7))
 (segment (start 9.178574 3.7) (end 9.178574 2.300003) (width 0.3) (layer "B.Cu") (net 7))
 (segment (start 7.362 1.671) (end 8.629 1.671) (width 0.25) (layer "F.Cu") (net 5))
 (segment (start 11.964287 3.228574) (end 11.035713 2.3) (width 0.25) (layer "F.Cu") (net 5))
 (segment (start 11.964287 3.7) (end 11.964287 3.228574) (width 0.25) (layer "F.Cu") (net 5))
 (segment (start 8.92179 1.716) (end 8.92327 1.71452) (width 0.25) (layer "F.Cu") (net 5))
 (segment (start 8.641 1.683) (end 8.674 1.716) (width 0.25) (layer "F.Cu") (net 5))
 (segment (start 5.708 2.5) (end 6.533 2.5) (width 0.25) (layer "F.Cu") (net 5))
 (segment (start 8.629 1.671) (end 8.641 1.683) (width 0.25) (layer "F.Cu") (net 5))
 (segment (start 8.674 1.716) (end 8.92179 1.716) (width 0.25) (layer "F.Cu") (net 5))
 (segment (start 8.92327 1.71452) (end 8.641 1.683) (width 0.25) (layer "F.Cu") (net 5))
 (segment (start 5.25 2.958) (end 5.708 2.5) (width 0.25) (layer "F.Cu") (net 5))
 (segment (start 7.327521 1.705479) (end 10.441192 1.705479) (width 0.25) (layer "F.Cu") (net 5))
 (segment (start 10.441192 1.705479) (end 11.035713 2.3) (width 0.25) (layer "F.Cu") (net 5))
 (segment (start 6.533 2.5) (end 7.327521 1.705479) (width 0.25) (layer "F.Cu") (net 5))
 (segment (start 6.533 2.5) (end 7.362 1.671) (width 0.25) (layer "F.Cu") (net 5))
 (via (at 5.25 2.958) (size 0.6) (drill 0.3) (layers "F.Cu" "B.Cu") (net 5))
 (segment (start 5.808 4.5) (end 5.229 3.921) (width 0.25) (layer "B.Cu") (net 5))
 (segment (start 5.229 2.979) (end 5.25 2.958) (width 0.25) (layer "B.Cu") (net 5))
 (segment (start 6.533 4.5) (end 5.808 4.5) (width 0.25) (layer "B.Cu") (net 5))
 (segment (start 5.229 3.921) (end 5.229 2.979) (width 0.25) (layer "B.Cu") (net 5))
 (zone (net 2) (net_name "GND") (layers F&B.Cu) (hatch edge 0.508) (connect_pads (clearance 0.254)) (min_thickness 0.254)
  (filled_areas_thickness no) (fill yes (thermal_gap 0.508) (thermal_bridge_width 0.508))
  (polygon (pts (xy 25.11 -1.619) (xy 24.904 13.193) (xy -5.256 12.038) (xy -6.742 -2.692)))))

